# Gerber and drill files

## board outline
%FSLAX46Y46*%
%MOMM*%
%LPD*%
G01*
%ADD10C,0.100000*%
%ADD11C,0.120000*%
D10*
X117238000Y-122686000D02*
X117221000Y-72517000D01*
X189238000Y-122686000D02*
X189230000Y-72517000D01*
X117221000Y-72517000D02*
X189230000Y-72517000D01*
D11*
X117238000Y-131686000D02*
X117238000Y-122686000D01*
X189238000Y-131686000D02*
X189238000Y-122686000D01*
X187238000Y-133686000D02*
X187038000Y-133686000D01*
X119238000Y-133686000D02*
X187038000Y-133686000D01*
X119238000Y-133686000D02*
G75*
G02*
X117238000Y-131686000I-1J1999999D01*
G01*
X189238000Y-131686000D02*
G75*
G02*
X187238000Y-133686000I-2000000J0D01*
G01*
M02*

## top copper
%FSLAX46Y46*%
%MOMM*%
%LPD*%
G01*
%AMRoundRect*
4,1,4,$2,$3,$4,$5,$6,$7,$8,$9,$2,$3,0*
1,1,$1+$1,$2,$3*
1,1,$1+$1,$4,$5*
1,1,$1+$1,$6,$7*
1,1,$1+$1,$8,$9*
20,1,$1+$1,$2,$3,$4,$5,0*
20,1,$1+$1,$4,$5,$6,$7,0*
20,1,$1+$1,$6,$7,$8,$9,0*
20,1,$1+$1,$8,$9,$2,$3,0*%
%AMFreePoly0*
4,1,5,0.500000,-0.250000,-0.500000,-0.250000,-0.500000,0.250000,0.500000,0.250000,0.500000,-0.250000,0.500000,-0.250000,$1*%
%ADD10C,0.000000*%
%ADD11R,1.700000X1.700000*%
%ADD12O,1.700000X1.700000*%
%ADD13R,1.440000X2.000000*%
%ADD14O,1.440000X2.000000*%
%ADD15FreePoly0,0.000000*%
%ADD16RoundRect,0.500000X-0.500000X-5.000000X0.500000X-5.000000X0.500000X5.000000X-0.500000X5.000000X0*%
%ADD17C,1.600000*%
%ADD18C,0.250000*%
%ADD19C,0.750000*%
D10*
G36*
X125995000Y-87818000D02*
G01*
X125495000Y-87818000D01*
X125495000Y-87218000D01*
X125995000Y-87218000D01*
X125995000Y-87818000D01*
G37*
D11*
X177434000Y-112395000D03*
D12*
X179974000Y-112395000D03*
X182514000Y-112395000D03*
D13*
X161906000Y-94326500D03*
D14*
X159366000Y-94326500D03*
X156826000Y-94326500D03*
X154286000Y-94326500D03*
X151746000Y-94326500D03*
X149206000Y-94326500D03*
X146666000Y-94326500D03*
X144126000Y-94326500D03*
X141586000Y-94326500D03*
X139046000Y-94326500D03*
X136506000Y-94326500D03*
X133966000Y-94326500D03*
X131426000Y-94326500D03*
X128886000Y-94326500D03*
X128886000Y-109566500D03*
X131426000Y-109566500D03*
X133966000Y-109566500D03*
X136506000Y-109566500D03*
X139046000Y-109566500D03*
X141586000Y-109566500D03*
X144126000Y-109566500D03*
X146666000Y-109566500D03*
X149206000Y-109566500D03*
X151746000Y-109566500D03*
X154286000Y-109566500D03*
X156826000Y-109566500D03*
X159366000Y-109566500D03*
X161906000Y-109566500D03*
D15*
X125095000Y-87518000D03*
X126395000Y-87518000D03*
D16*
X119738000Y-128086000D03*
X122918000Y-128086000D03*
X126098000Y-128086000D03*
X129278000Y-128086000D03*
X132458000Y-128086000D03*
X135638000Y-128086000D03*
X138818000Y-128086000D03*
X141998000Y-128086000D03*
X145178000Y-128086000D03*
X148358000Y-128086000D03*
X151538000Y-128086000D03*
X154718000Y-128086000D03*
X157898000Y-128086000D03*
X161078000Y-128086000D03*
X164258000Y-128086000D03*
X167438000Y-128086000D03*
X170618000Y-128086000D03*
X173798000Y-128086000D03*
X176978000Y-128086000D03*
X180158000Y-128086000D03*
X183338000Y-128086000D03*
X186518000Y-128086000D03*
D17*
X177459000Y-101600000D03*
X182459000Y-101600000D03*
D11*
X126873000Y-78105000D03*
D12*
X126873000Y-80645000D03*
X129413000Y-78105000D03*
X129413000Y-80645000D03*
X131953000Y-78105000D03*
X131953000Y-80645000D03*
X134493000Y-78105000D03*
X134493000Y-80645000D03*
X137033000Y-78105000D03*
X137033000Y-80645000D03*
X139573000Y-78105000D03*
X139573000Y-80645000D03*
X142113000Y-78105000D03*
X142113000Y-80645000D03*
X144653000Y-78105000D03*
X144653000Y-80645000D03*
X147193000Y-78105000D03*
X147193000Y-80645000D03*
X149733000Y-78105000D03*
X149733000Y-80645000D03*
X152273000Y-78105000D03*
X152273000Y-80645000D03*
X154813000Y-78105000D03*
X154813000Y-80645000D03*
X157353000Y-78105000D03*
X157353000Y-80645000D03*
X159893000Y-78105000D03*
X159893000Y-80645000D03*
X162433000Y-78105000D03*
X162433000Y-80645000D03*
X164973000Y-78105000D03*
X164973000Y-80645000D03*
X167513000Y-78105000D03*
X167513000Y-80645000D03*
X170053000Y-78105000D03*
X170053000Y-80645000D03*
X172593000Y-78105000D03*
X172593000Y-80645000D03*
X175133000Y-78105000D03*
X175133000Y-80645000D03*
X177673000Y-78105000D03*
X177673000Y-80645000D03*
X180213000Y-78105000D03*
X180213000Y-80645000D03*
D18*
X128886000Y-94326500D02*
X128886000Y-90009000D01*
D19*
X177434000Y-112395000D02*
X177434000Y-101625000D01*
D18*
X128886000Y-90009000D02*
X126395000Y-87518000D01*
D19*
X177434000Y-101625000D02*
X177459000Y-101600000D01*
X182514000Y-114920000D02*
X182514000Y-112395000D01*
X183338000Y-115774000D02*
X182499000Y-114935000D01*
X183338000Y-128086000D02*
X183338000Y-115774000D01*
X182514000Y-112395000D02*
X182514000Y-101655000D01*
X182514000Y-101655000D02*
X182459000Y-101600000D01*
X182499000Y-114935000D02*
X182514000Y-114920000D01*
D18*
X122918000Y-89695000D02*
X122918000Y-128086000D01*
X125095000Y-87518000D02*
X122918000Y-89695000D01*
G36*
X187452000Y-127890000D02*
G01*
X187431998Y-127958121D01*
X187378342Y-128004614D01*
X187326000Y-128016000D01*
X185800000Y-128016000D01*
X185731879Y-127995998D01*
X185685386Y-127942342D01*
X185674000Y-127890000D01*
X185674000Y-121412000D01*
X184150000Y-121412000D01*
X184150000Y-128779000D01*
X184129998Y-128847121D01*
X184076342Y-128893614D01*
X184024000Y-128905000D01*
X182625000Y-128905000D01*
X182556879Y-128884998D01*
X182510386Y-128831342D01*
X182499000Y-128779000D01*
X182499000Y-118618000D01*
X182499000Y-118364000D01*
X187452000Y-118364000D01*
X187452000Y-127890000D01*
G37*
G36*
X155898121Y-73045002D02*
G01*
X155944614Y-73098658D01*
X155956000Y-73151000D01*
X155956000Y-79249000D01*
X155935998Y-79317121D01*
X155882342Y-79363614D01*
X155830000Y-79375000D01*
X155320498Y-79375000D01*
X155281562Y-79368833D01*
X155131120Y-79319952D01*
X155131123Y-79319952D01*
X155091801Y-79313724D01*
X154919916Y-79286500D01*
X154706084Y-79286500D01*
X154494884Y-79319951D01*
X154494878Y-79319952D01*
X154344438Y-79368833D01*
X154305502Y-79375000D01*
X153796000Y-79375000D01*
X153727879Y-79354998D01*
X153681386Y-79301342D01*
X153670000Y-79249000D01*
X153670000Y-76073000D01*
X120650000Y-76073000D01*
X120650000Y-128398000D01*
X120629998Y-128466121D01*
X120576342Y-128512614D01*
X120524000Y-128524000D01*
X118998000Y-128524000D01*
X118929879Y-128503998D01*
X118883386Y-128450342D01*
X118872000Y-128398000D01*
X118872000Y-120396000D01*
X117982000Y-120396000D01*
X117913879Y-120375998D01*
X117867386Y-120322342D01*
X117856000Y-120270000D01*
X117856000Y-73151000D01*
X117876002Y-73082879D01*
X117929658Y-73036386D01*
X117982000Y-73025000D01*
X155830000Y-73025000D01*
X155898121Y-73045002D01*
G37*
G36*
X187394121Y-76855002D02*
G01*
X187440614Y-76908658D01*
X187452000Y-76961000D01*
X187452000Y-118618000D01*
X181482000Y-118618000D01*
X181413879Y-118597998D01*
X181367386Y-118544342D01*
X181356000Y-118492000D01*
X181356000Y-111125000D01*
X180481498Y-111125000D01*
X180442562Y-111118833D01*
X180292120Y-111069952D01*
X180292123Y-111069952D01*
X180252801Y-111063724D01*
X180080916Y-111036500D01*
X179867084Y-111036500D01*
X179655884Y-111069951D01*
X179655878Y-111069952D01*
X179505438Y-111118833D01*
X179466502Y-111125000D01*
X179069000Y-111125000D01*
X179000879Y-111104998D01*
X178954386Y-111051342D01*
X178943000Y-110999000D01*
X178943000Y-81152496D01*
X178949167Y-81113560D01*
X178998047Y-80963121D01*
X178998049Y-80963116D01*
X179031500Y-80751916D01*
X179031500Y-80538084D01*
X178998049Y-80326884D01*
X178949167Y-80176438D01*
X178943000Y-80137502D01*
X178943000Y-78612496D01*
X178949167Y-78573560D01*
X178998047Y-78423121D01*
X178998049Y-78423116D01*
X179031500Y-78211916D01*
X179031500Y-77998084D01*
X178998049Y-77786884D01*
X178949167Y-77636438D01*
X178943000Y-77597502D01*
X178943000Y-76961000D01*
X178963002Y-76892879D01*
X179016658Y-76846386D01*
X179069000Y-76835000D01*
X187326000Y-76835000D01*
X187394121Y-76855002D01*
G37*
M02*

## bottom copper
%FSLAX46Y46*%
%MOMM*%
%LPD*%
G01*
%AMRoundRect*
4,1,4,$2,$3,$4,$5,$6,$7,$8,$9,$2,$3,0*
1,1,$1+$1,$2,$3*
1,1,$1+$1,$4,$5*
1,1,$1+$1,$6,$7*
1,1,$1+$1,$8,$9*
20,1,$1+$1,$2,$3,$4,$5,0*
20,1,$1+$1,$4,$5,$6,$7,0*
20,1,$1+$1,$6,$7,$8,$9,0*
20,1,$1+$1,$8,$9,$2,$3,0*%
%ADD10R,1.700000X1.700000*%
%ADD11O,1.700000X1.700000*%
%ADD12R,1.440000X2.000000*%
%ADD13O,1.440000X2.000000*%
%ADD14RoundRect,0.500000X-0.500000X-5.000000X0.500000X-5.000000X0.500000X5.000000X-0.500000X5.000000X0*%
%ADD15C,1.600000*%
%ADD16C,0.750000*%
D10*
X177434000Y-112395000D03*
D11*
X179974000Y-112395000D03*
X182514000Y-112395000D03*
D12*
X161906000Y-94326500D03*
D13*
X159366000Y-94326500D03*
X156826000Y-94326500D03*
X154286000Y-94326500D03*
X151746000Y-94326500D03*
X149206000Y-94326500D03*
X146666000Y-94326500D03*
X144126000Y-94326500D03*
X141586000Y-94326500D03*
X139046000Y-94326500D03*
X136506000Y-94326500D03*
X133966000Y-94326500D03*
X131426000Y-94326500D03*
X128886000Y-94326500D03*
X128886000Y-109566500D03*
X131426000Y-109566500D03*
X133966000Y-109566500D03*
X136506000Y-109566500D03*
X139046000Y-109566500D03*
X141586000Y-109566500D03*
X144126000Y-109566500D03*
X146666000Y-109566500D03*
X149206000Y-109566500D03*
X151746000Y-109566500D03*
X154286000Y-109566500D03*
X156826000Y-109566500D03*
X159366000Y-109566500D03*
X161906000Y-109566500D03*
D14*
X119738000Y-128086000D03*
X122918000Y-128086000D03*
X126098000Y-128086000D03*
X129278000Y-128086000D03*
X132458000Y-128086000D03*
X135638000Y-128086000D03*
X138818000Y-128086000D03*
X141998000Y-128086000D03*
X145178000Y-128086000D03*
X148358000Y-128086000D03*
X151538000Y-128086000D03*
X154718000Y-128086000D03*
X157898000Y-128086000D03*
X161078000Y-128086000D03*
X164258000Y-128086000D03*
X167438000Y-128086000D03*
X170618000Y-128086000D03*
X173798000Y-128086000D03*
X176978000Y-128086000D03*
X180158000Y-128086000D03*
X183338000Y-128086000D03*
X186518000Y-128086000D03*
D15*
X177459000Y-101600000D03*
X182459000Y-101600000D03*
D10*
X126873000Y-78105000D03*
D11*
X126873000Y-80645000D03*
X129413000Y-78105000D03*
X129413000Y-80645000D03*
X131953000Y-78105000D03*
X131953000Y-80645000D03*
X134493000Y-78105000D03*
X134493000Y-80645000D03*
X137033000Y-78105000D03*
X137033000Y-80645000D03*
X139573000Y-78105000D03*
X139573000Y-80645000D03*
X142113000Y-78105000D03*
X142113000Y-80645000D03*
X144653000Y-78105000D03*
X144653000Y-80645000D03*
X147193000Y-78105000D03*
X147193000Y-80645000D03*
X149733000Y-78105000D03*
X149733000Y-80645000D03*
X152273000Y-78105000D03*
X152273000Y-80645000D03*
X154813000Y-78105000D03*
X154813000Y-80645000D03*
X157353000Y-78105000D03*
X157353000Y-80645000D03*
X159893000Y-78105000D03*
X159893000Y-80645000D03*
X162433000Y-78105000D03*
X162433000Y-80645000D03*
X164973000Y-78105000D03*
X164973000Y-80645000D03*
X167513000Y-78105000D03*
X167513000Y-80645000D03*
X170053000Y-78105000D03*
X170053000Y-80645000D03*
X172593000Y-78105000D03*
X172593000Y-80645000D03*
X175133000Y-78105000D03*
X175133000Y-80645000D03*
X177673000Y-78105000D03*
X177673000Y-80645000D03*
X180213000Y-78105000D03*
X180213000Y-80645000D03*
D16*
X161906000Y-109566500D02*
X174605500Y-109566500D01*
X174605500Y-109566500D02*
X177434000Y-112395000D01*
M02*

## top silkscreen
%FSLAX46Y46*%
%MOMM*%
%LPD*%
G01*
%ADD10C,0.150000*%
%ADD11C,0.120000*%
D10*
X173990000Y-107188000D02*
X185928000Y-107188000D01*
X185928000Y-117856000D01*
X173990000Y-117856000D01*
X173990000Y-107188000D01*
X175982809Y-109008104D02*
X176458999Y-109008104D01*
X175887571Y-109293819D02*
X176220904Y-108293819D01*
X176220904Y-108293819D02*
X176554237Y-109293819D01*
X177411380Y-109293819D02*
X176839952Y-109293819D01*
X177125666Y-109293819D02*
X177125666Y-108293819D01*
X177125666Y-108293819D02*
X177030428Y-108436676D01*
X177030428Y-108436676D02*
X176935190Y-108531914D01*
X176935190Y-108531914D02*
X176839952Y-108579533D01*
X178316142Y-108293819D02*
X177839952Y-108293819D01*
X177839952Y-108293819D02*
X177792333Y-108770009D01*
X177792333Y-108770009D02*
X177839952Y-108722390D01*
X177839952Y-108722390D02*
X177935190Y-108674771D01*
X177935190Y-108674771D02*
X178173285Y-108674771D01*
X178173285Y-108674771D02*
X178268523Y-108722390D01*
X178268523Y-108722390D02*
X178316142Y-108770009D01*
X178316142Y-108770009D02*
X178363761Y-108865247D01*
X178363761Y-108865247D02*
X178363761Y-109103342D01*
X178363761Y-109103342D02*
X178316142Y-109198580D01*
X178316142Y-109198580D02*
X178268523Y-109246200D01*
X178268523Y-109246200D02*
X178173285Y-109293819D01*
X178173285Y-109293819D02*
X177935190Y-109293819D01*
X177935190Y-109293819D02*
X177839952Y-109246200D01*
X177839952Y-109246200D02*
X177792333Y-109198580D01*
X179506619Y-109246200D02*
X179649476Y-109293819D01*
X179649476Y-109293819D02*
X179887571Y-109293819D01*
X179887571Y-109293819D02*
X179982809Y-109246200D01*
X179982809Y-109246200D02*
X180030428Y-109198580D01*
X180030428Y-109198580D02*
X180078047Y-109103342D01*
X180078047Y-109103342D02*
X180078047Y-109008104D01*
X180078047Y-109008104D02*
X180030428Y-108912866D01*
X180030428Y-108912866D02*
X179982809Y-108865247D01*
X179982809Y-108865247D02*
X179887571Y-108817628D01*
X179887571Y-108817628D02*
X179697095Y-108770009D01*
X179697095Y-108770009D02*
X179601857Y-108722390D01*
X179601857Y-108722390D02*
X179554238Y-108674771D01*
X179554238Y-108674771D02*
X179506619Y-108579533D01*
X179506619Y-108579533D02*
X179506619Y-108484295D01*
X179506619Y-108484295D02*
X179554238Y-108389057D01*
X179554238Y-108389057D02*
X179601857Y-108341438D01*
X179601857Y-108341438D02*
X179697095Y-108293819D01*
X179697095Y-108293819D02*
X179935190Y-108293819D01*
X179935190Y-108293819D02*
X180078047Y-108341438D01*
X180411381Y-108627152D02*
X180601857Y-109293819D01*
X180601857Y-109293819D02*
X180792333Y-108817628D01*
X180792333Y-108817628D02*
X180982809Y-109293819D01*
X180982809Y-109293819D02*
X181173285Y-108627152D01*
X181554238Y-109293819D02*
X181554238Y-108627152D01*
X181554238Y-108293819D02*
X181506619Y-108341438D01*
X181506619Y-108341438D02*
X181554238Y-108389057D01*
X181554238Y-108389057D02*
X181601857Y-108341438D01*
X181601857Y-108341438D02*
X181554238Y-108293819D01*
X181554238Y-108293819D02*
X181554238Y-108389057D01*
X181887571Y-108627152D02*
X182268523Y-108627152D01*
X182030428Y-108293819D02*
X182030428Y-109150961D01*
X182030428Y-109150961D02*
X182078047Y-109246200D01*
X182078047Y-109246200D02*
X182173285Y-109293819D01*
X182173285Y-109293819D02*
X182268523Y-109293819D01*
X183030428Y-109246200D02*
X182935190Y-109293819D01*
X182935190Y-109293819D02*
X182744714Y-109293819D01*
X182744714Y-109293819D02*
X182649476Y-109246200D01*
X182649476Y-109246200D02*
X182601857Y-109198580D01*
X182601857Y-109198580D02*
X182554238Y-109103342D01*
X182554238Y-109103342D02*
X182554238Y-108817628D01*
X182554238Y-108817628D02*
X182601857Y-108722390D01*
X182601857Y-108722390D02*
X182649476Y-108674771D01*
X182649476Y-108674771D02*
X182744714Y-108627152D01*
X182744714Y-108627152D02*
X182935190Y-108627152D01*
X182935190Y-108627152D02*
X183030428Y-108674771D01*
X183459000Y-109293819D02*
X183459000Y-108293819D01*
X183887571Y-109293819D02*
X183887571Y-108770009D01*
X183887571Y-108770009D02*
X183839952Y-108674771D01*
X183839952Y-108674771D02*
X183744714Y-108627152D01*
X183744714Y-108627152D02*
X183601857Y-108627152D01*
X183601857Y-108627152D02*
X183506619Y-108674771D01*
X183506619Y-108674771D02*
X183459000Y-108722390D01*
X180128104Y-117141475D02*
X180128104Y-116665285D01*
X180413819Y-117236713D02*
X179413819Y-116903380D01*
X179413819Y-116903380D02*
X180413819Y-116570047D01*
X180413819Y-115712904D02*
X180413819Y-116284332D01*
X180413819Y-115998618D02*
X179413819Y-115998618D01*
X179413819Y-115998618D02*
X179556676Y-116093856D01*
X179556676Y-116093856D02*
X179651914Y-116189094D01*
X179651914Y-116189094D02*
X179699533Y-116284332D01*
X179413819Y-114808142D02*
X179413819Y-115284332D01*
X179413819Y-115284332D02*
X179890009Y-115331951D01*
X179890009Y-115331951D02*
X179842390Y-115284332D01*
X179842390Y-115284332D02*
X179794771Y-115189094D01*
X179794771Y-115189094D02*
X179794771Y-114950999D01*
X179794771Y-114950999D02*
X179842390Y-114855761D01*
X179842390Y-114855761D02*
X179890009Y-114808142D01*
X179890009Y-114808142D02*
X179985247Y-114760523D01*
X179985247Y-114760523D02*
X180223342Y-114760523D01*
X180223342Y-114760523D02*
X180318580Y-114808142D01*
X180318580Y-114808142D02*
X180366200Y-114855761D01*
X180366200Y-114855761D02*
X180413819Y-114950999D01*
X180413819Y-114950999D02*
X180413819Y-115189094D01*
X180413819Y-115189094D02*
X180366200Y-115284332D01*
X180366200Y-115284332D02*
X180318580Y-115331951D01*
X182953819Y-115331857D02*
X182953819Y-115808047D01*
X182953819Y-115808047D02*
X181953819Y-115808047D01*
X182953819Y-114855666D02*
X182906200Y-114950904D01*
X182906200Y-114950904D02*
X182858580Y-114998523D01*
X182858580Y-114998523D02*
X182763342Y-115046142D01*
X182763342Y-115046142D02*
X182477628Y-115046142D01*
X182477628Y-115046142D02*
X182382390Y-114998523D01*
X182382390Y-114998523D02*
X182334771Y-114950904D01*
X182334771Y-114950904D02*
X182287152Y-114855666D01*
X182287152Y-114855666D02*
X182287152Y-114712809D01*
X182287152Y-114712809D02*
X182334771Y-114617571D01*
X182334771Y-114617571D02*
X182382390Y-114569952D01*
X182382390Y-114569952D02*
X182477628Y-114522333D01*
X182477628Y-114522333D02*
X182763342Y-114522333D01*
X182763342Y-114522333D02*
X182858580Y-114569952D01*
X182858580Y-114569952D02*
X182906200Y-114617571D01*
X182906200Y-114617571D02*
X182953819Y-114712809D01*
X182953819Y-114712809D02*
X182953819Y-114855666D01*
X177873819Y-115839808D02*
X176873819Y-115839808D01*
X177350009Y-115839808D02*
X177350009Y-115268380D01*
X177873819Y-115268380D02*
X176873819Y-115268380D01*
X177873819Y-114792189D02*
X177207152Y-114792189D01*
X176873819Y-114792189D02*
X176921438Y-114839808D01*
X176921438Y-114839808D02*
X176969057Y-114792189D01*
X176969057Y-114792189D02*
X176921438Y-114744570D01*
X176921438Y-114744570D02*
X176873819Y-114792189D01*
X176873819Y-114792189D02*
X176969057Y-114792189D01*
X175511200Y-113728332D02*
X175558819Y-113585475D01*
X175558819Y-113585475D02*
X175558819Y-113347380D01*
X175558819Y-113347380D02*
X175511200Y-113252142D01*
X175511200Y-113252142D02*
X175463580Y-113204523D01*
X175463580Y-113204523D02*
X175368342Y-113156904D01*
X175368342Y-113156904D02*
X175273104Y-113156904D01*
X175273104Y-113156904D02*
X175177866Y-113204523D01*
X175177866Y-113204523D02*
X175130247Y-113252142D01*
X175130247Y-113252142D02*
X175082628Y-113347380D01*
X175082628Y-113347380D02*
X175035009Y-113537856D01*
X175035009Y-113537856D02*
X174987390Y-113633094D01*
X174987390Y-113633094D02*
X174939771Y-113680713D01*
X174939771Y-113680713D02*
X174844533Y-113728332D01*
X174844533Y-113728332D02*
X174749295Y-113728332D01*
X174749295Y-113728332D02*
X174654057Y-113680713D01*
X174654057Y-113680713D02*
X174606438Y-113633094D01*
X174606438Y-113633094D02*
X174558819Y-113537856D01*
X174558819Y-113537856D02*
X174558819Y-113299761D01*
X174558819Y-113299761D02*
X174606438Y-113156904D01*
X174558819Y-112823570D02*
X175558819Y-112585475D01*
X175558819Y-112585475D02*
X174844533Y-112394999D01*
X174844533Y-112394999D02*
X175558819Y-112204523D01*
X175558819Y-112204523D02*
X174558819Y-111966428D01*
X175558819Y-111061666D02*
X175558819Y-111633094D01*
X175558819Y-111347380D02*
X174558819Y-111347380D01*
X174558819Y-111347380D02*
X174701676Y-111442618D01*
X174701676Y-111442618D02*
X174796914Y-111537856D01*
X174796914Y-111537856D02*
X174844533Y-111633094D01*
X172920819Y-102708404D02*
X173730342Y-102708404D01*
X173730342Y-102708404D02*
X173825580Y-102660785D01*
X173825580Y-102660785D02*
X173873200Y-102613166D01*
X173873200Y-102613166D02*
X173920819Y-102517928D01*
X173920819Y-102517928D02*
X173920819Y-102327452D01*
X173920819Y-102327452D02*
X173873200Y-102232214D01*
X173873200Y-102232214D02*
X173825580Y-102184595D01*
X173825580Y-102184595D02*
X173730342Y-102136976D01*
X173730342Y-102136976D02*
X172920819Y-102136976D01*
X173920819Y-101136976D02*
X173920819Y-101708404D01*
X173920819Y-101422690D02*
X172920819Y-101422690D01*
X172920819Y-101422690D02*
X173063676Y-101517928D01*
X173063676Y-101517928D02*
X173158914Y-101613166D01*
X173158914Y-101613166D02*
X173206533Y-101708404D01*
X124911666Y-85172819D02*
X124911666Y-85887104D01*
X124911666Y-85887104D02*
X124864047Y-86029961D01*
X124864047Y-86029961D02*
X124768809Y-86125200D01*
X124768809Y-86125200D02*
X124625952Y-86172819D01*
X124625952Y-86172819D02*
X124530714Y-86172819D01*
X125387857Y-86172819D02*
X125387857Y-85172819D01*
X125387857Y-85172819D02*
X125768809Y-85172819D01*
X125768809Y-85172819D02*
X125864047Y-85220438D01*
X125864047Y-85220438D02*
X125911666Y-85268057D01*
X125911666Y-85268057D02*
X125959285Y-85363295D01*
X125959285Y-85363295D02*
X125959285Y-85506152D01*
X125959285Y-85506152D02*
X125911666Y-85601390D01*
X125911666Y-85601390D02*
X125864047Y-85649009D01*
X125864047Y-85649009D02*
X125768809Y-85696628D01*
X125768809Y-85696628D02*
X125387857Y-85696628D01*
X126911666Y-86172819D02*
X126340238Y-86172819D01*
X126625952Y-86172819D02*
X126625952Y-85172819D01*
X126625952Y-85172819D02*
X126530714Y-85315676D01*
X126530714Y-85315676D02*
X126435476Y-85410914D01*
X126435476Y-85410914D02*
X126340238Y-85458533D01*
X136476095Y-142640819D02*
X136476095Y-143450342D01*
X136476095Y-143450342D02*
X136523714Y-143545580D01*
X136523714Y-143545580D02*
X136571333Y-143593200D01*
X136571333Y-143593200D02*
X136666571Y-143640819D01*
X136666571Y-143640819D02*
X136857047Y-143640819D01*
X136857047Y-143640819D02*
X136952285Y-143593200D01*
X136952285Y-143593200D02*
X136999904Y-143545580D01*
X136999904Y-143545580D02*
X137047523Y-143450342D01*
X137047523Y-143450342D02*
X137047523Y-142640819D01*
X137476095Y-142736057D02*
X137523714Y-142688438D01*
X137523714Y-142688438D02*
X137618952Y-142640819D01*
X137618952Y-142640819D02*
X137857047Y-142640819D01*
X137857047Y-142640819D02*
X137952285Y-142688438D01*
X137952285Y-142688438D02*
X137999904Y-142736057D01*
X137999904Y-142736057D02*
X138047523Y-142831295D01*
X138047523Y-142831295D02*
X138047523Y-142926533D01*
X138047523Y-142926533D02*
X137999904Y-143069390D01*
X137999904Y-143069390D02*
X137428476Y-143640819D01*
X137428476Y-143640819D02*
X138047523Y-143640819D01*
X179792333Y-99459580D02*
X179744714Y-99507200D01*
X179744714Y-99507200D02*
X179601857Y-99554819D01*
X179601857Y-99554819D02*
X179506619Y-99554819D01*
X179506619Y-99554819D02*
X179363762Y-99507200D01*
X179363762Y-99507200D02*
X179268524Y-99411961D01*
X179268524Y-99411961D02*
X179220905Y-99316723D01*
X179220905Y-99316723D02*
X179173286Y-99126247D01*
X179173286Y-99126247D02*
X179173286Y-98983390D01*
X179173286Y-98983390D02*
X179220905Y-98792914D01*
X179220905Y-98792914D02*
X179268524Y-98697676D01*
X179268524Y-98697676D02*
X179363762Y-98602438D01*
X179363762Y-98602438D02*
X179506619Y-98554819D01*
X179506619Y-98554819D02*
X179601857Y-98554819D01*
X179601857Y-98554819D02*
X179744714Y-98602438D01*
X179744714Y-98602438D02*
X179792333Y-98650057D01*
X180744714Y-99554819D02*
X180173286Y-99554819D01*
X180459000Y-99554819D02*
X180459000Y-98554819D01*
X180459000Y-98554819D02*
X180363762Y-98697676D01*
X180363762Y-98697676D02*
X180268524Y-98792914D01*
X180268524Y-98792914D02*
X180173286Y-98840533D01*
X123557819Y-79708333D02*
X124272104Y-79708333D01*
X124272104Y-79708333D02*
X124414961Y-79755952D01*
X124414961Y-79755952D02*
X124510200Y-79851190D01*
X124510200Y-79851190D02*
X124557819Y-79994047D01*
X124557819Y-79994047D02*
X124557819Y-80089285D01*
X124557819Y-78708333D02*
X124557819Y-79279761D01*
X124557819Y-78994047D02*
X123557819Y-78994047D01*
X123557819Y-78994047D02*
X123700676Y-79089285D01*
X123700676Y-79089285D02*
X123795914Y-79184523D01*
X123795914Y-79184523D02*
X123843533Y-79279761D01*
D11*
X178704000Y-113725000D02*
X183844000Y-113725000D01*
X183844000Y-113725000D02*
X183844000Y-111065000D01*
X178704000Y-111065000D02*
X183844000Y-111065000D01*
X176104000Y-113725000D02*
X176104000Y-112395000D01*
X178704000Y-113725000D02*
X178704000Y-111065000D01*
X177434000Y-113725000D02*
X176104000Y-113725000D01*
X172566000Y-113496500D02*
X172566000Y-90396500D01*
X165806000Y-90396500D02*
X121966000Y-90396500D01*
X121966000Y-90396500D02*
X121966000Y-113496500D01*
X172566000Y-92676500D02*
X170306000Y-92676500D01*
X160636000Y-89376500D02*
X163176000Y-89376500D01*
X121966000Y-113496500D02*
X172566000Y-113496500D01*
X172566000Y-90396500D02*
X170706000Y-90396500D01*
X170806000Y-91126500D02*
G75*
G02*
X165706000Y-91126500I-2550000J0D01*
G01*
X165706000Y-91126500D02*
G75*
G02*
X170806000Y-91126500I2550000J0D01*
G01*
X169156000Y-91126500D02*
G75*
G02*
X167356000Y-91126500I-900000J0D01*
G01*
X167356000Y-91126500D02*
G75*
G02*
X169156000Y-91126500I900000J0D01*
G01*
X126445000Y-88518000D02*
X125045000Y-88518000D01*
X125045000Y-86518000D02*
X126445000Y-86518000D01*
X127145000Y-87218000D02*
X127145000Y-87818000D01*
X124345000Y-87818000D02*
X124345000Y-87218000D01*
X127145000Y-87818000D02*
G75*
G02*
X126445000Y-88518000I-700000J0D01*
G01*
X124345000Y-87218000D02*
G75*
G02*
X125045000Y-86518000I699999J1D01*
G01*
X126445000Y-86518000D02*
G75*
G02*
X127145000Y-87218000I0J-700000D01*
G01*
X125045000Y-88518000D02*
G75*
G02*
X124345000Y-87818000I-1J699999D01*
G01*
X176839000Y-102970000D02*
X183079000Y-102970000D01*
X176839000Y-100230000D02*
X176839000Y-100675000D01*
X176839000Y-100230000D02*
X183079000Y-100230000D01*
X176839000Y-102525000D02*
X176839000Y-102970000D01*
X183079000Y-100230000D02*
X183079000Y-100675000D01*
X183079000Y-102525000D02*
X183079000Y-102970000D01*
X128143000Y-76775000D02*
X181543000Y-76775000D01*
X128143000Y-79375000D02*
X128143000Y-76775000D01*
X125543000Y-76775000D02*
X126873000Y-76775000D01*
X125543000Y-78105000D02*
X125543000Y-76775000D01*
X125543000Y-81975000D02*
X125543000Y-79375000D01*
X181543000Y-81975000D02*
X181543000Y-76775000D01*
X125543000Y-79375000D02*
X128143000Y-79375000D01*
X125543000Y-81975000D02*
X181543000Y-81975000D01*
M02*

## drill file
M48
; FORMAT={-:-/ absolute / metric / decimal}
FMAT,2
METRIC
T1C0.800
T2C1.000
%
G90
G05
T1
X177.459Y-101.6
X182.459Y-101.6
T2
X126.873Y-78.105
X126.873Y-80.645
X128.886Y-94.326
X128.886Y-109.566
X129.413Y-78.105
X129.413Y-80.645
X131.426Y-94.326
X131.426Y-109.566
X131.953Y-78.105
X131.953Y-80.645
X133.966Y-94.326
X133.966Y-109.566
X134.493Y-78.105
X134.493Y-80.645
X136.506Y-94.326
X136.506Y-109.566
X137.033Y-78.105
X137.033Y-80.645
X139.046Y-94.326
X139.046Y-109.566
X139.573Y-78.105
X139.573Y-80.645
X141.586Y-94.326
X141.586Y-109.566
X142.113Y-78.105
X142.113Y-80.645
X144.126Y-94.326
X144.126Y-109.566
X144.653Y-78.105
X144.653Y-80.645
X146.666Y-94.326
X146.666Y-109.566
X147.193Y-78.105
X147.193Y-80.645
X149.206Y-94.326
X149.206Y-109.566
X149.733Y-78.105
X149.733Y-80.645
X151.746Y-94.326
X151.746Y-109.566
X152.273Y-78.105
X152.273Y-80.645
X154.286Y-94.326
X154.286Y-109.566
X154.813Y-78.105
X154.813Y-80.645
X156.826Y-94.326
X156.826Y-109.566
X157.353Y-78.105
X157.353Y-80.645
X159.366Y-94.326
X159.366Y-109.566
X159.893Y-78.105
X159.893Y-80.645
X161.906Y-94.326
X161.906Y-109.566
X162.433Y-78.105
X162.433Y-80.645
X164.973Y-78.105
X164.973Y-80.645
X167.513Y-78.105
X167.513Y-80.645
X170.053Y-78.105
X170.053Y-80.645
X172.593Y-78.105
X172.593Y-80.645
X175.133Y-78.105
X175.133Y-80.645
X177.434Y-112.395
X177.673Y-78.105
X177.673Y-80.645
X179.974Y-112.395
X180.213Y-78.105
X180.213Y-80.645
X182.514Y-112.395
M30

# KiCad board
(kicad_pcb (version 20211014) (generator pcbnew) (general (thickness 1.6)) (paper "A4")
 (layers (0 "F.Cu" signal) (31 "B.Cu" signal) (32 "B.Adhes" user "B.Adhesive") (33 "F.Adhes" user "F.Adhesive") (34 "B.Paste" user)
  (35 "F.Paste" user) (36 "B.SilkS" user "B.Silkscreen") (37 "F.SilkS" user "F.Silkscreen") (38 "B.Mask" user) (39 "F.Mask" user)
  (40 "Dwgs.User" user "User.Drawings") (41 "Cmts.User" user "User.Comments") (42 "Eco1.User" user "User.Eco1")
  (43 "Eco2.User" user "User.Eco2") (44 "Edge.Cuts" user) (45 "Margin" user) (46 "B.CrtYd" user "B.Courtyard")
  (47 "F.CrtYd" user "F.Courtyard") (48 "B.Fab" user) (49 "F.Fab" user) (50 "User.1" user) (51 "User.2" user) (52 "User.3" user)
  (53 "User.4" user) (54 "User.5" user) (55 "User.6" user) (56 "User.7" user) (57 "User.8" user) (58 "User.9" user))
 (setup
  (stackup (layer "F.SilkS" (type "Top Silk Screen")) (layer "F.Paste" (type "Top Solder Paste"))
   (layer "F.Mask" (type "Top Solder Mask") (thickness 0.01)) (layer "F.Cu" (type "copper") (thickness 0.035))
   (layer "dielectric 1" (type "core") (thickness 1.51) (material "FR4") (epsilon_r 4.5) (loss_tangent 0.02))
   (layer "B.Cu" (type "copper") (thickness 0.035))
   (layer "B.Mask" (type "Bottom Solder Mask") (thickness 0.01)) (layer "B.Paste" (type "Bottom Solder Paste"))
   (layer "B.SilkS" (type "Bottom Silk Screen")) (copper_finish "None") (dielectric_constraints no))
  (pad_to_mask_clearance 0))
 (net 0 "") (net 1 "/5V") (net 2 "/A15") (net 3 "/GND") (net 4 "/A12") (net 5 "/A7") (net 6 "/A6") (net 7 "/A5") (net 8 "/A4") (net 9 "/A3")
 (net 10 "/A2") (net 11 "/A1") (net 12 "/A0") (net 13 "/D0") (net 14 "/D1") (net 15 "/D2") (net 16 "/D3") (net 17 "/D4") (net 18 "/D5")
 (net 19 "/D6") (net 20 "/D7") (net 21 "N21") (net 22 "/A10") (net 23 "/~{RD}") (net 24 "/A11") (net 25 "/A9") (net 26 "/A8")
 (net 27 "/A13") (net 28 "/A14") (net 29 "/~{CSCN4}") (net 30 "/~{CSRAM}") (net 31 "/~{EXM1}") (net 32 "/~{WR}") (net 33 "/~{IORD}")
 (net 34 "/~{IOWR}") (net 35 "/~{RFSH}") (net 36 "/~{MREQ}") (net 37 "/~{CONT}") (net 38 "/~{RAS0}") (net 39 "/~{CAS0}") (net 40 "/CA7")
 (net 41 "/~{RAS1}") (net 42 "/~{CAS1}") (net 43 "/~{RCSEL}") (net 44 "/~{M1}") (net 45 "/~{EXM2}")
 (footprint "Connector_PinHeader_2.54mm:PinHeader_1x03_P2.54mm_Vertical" (layer "F.Cu") (at 177.434 112.395 90)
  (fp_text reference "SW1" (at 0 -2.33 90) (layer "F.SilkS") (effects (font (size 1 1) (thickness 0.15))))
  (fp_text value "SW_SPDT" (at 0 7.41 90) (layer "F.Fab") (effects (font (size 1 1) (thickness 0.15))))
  (fp_line (start -1.33 1.27) (end -1.33 6.41) (layer "F.SilkS") (width 0.12))
  (fp_line (start -1.33 6.41) (end 1.33 6.41) (layer "F.SilkS") (width 0.12))
  (fp_line (start 1.33 1.27) (end 1.33 6.41) (layer "F.SilkS") (width 0.12))
  (fp_line (start -1.33 -1.33) (end 0 -1.33) (layer "F.SilkS") (width 0.12))
  (fp_line (start -1.33 1.27) (end 1.33 1.27) (layer "F.SilkS") (width 0.12))
  (fp_line (start -1.33 0) (end -1.33 -1.33) (layer "F.SilkS") (width 0.12))
  (pad "1" thru_hole rect (at 0 0 90) (size 1.7 1.7) (drill 1) (layers *.Cu *.Mask) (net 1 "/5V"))
  (pad "2" thru_hole oval (at 0 2.54 90) (size 1.7 1.7) (drill 1) (layers *.Cu *.Mask) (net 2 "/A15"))
  (pad "3" thru_hole oval (at 0 5.08 90) (size 1.7 1.7) (drill 1) (layers *.Cu *.Mask) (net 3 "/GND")))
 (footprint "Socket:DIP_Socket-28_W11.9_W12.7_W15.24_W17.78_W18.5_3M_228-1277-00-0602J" (layer "F.Cu") (at 161.906 94.3265 -90)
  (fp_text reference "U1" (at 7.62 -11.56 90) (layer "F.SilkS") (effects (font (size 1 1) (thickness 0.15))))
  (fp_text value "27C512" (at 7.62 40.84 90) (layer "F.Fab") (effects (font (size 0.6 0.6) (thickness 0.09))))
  (fp_line (start 19.17 -10.66) (end -3.93 -10.66) (layer "F.SilkS") (width 0.12))
  (fp_line (start -3.93 -3.9) (end -3.93 39.94) (layer "F.SilkS") (width 0.12))
  (fp_line (start -3.93 39.94) (end 19.17 39.94) (layer "F.SilkS") (width 0.12))
  (fp_line (start -1.65 -10.66) (end -1.65 -8.4) (layer "F.SilkS") (width 0.12))
  (fp_line (start -4.95 1.27) (end -4.95 -1.27) (layer "F.SilkS") (width 0.12))
  (fp_line (start 19.17 39.94) (end 19.17 -10.66) (layer "F.SilkS") (width 0.12))
  (fp_line (start -3.93 -10.66) (end -3.93 -8.8) (layer "F.SilkS") (width 0.12))
  (fp_circle (center -3.2 -6.35) (end -0.65 -6.35) (layer "F.SilkS") (width 0.12) (fill none))
  (fp_circle (center -3.2 -6.35) (end -2.3 -6.35) (layer "F.SilkS") (width 0.12) (fill none))
  (pad "1" thru_hole rect (at 0 0 270) (size 2 1.44) (drill 1) (layers *.Cu *.Mask) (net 2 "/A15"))
  (pad "2" thru_hole oval (at 0 2.54 270) (size 2 1.44) (drill 1) (layers *.Cu *.Mask) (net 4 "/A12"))
  (pad "3" thru_hole oval (at 0 5.08 270) (size 2 1.44) (drill 1) (layers *.Cu *.Mask) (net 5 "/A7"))
  (pad "4" thru_hole oval (at 0 7.62 270) (size 2 1.44) (drill 1) (layers *.Cu *.Mask) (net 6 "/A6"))
  (pad "5" thru_hole oval (at 0 10.16 270) (size 2 1.44) (drill 1) (layers *.Cu *.Mask) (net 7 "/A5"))
  (pad "6" thru_hole oval (at 0 12.7 270) (size 2 1.44) (drill 1) (layers *.Cu *.Mask) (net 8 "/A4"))
  (pad "7" thru_hole oval (at 0 15.24 270) (size 2 1.44) (drill 1) (layers *.Cu *.Mask) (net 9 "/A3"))
  (pad "8" thru_hole oval (at 0 17.78 270) (size 2 1.44) (drill 1) (layers *.Cu *.Mask) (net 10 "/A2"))
  (pad "9" thru_hole oval (at 0 20.32 270) (size 2 1.44) (drill 1) (layers *.Cu *.Mask) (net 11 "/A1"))
  (pad "10" thru_hole oval (at 0 22.86 270) (size 2 1.44) (drill 1) (layers *.Cu *.Mask) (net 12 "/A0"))
  (pad "11" thru_hole oval (at 0 25.4 270) (size 2 1.44) (drill 1) (layers *.Cu *.Mask) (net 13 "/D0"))
  (pad "12" thru_hole oval (at 0 27.94 270) (size 2 1.44) (drill 1) (layers *.Cu *.Mask) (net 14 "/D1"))
  (pad "13" thru_hole oval (at 0 30.48 270) (size 2 1.44) (drill 1) (layers *.Cu *.Mask) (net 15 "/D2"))
  (pad "14" thru_hole oval (at 0 33.02 270) (size 2 1.44) (drill 1) (layers *.Cu *.Mask) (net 3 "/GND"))
  (pad "15" thru_hole oval (at 15.24 33.02 270) (size 2 1.44) (drill 1) (layers *.Cu *.Mask) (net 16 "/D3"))
  (pad "16" thru_hole oval (at 15.24 30.48 270) (size 2 1.44) (drill 1) (layers *.Cu *.Mask) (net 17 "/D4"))
  (pad "17" thru_hole oval (at 15.24 27.94 270) (size 2 1.44) (drill 1) (layers *.Cu *.Mask) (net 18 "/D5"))
  (pad "18" thru_hole oval (at 15.24 25.4 270) (size 2 1.44) (drill 1) (layers *.Cu *.Mask) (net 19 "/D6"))
  (pad "19" thru_hole oval (at 15.24 22.86 270) (size 2 1.44) (drill 1) (layers *.Cu *.Mask) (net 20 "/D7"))
  (pad "20" thru_hole oval (at 15.24 20.32 270) (size 2 1.44) (drill 1) (layers *.Cu *.Mask) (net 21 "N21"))
  (pad "21" thru_hole oval (at 15.24 17.78 270) (size 2 1.44) (drill 1) (layers *.Cu *.Mask) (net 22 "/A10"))
  (pad "22" thru_hole oval (at 15.24 15.24 270) (size 2 1.44) (drill 1) (layers *.Cu *.Mask) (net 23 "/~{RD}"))
  (pad "23" thru_hole oval (at 15.24 12.7 270) (size 2 1.44) (drill 1) (layers *.Cu *.Mask) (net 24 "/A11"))
  (pad "24" thru_hole oval (at 15.24 10.16 270) (size 2 1.44) (drill 1) (layers *.Cu *.Mask) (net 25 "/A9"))
  (pad "25" thru_hole oval (at 15.24 7.62 270) (size 2 1.44) (drill 1) (layers *.Cu *.Mask) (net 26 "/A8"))
  (pad "26" thru_hole oval (at 15.24 5.08 270) (size 2 1.44) (drill 1) (layers *.Cu *.Mask) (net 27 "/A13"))
  (pad "27" thru_hole oval (at 15.24 2.54 270) (size 2 1.44) (drill 1) (layers *.Cu *.Mask) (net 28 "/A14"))
  (pad "28" thru_hole oval (at 15.24 0 270) (size 2 1.44) (drill 1) (layers *.Cu *.Mask) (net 1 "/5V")))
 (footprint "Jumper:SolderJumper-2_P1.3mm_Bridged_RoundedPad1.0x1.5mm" (layer "F.Cu") (at 125.745 87.518)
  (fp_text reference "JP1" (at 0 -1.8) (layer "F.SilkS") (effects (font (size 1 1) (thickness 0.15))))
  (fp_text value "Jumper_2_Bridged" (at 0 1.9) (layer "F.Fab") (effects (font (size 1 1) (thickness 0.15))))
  (fp_poly (pts (xy 0.25 -0.3) (xy -0.25 -0.3) (xy -0.25 0.3) (xy 0.25 0.3)) (layer "F.Cu") (width 0) (fill solid))
  (fp_line (start 0.7 1) (end -0.7 1) (layer "F.SilkS") (width 0.12))
  (fp_line (start -0.7 -1) (end 0.7 -1) (layer "F.SilkS") (width 0.12))
  (fp_line (start 1.4 -0.3) (end 1.4 0.3) (layer "F.SilkS") (width 0.12))
  (fp_line (start -1.4 0.3) (end -1.4 -0.3) (layer "F.SilkS") (width 0.12))
  (fp_arc (start 1.4 0.3) (mid 1.194975 0.794975) (end 0.7 1) (layer "F.SilkS") (width 0.12))
  (fp_arc (start -1.4 -0.3) (mid -1.194975 -0.794975) (end -0.7 -1) (layer "F.SilkS") (width 0.12))
  (fp_arc (start 0.7 -1) (mid 1.194975 -0.794975) (end 1.4 -0.3) (layer "F.SilkS") (width 0.12))
  (fp_arc (start -0.7 1) (mid -1.194975 0.794975) (end -1.4 0.3) (layer "F.SilkS") (width 0.12))
  (pad "1" smd custom (at -0.65 0) (size 1 0.5) (layers "F.Cu" "F.Mask") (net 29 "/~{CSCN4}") (zone_connect 2)
   (options (clearance outline) (anchor rect)) (primitives))
  (pad "2" smd custom (at 0.65 0) (size 1 0.5) (layers "F.Cu" "F.Mask") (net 1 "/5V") (zone_connect 2)
   (options (clearance outline) (anchor rect)) (primitives)))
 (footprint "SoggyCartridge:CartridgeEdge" (layer "F.Cu") (at 120.138 122.586)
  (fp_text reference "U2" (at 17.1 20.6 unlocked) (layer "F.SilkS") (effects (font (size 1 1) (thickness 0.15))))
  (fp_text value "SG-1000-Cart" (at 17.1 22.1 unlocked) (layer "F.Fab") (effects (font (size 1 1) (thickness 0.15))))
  (fp_line (start -2.9 9.1) (end -2.9 0.1) (layer "Edge.Cuts") (width 0.12))
  (fp_line (start 69.1 9.1) (end 69.1 0.1) (layer "Edge.Cuts") (width 0.12))
  (fp_line (start 67.1 11.1) (end 66.9 11.1) (layer "Edge.Cuts") (width 0.12))
  (fp_line (start -0.9 11.1) (end 66.9 11.1) (layer "Edge.Cuts") (width 0.12))
  (fp_arc (start -0.9 11.1) (mid -2.314214 10.514214) (end -2.9 9.1) (layer "Edge.Cuts") (width 0.12))
  (fp_arc (start 69.1 9.1) (mid 68.514214 10.514214) (end 67.1 11.1) (layer "Edge.Cuts") (width 0.12))
  (pad "A1" connect roundrect (at -0.4 5.5) (size 2 11) (layers "B.Cu" "B.Mask") (roundrect_rratio 0.25) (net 12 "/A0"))
  (pad "A2" connect roundrect (at 2.78 5.5) (size 2 11) (layers "B.Cu" "B.Mask") (roundrect_rratio 0.25) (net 11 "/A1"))
  (pad "A3" connect roundrect (at 5.96 5.5) (size 2 11) (layers "B.Cu" "B.Mask") (roundrect_rratio 0.25) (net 10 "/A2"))
  (pad "A4" connect roundrect (at 9.14 5.5) (size 2 11) (layers "B.Cu" "B.Mask") (roundrect_rratio 0.25) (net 9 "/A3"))
  (pad "A5" connect roundrect (at 12.32 5.5) (size 2 11) (layers "B.Cu" "B.Mask") (roundrect_rratio 0.25) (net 8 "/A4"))
  (pad "A6" connect roundrect (at 15.5 5.5) (size 2 11) (layers "B.Cu" "B.Mask") (roundrect_rratio 0.25) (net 7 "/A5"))
  (pad "A7" connect roundrect (at 18.68 5.5) (size 2 11) (layers "B.Cu" "B.Mask") (roundrect_rratio 0.25) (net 6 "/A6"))
  (pad "A8" connect roundrect (at 21.86 5.5) (size 2 11) (layers "B.Cu" "B.Mask") (roundrect_rratio 0.25) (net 5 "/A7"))
  (pad "A9" connect roundrect (at 25.04 5.5) (size 2 11) (layers "B.Cu" "B.Mask") (roundrect_rratio 0.25) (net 26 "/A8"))
  (pad "A10" connect roundrect (at 28.22 5.5) (size 2 11) (layers "B.Cu" "B.Mask") (roundrect_rratio 0.25) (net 25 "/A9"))
  (pad "A11" connect roundrect (at 31.4 5.5) (size 2 11) (layers "B.Cu" "B.Mask") (roundrect_rratio 0.25) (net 22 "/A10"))
  (pad "A12" connect roundrect (at 34.58 5.5) (size 2 11) (layers "B.Cu" "B.Mask") (roundrect_rratio 0.25) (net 24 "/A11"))
  (pad "A13" connect roundrect (at 37.76 5.5) (size 2 11) (layers "B.Cu" "B.Mask") (roundrect_rratio 0.25) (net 4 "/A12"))
  (pad "A14" connect roundrect (at 40.94 5.5) (size 2 11) (layers "B.Cu" "B.Mask") (roundrect_rratio 0.25) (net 27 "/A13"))
  (pad "A15" connect roundrect (at 44.12 5.5) (size 2 11) (layers "B.Cu" "B.Mask") (roundrect_rratio 0.25) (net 13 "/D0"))
  (pad "A16" connect roundrect (at 47.3 5.5) (size 2 11) (layers "B.Cu" "B.Mask") (roundrect_rratio 0.25) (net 14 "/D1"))
  (pad "A17" connect roundrect (at 50.48 5.5) (size 2 11) (layers "B.Cu" "B.Mask") (roundrect_rratio 0.25) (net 15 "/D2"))
  (pad "A18" connect roundrect (at 53.66 5.5) (size 2 11) (layers "B.Cu" "B.Mask") (roundrect_rratio 0.25) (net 16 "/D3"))
  (pad "A19" connect roundrect (at 56.84 5.5) (size 2 11) (layers "B.Cu" "B.Mask") (roundrect_rratio 0.25) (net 17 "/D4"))
  (pad "A20" connect roundrect (at 60.02 5.5) (size 2 11) (layers "B.Cu" "B.Mask") (roundrect_rratio 0.25) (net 18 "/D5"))
  (pad "A21" connect roundrect (at 63.2 5.5) (size 2 11) (layers "B.Cu" "B.Mask") (roundrect_rratio 0.25) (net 19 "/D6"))
  (pad "A22" connect roundrect (at 66.38 5.5) (size 2 11) (layers "B.Cu" "B.Mask") (roundrect_rratio 0.25) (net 20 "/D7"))
  (pad "B1" connect roundrect (at -0.4 5.5) (size 2 11) (layers "F.Cu" "F.Mask") (roundrect_rratio 0.25) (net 1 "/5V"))
  (pad "B2" connect roundrect (at 2.78 5.5) (size 2 11) (layers "F.Cu" "F.Mask") (roundrect_rratio 0.25) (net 29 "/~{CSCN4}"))
  (pad "B3" connect roundrect (at 5.96 5.5) (size 2 11) (layers "F.Cu" "F.Mask") (roundrect_rratio 0.25) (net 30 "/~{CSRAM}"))
  (pad "B4" connect roundrect (at 9.14 5.5) (size 2 11) (layers "F.Cu" "F.Mask") (roundrect_rratio 0.25) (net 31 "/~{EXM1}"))
  (pad "B5" connect roundrect (at 12.32 5.5) (size 2 11) (layers "F.Cu" "F.Mask") (roundrect_rratio 0.25) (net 23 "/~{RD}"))
  (pad "B6" connect roundrect (at 15.5 5.5) (size 2 11) (layers "F.Cu" "F.Mask") (roundrect_rratio 0.25) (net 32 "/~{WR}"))
  (pad "B7" connect roundrect (at 18.68 5.5) (size 2 11) (layers "F.Cu" "F.Mask") (roundrect_rratio 0.25) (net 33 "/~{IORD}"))
  (pad "B8" connect roundrect (at 21.86 5.5) (size 2 11) (layers "F.Cu" "F.Mask") (roundrect_rratio 0.25) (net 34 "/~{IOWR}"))
  (pad "B9" connect roundrect (at 25.04 5.5) (size 2 11) (layers "F.Cu" "F.Mask") (roundrect_rratio 0.25) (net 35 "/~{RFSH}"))
  (pad "B10" connect roundrect (at 28.22 5.5) (size 2 11) (layers "F.Cu" "F.Mask") (roundrect_rratio 0.25) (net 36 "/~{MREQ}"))
  (pad "B11" connect roundrect (at 31.4 5.5) (size 2 11) (layers "F.Cu" "F.Mask") (roundrect_rratio 0.25) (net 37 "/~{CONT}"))
  (pad "B12" connect roundrect (at 34.58 5.5) (size 2 11) (layers "F.Cu" "F.Mask") (roundrect_rratio 0.25) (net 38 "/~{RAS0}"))
  (pad "B13" connect roundrect (at 37.76 5.5) (size 2 11) (layers "F.Cu" "F.Mask") (roundrect_rratio 0.25) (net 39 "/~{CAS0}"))
  (pad "B14" connect roundrect (at 40.94 5.5) (size 2 11) (layers "F.Cu" "F.Mask") (roundrect_rratio 0.25) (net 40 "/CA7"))
  (pad "B15" connect roundrect (at 44.12 5.5) (size 2 11) (layers "F.Cu" "F.Mask") (roundrect_rratio 0.25) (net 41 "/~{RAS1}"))
  (pad "B16" connect roundrect (at 47.3 5.5) (size 2 11) (layers "F.Cu" "F.Mask") (roundrect_rratio 0.25) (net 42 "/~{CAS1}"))
  (pad "B17" connect roundrect (at 50.48 5.5) (size 2 11) (layers "F.Cu" "F.Mask") (roundrect_rratio 0.25) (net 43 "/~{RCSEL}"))
  (pad "B18" connect roundrect (at 53.66 5.5) (size 2 11) (layers "F.Cu" "F.Mask") (roundrect_rratio 0.25) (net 28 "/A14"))
  (pad "B19" connect roundrect (at 56.84 5.5) (size 2 11) (layers "F.Cu" "F.Mask") (roundrect_rratio 0.25) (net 21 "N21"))
  (pad "B20" connect roundrect (at 60.02 5.5) (size 2 11) (layers "F.Cu" "F.Mask") (roundrect_rratio 0.25) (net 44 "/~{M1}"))
  (pad "B21" connect roundrect (at 63.2 5.5) (size 2 11) (layers "F.Cu" "F.Mask") (roundrect_rratio 0.25) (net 3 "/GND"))
  (pad "B22" connect roundrect (at 66.38 5.5) (size 2 11) (layers "F.Cu" "F.Mask") (roundrect_rratio 0.25) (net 3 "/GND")))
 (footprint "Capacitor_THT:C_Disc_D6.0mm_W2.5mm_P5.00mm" (layer "F.Cu") (at 177.459 101.6)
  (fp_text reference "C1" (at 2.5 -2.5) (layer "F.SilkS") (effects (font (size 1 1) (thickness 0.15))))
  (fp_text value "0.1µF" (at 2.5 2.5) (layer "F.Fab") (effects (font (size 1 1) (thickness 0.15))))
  (fp_line (start -0.62 1.37) (end 5.62 1.37) (layer "F.SilkS") (width 0.12))
  (fp_line (start -0.62 -1.37) (end -0.62 -0.925) (layer "F.SilkS") (width 0.12))
  (fp_line (start -0.62 -1.37) (end 5.62 -1.37) (layer "F.SilkS") (width 0.12))
  (fp_line (start -0.62 0.925) (end -0.62 1.37) (layer "F.SilkS") (width 0.12))
  (fp_line (start 5.62 -1.37) (end 5.62 -0.925) (layer "F.SilkS") (width 0.12))
  (fp_line (start 5.62 0.925) (end 5.62 1.37) (layer "F.SilkS") (width 0.12))
  (pad "1" thru_hole circle (at 0 0) (size 1.6 1.6) (drill 0.8) (layers *.Cu *.Mask) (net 1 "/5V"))
  (pad "2" thru_hole circle (at 5 0) (size 1.6 1.6) (drill 0.8) (layers *.Cu *.Mask) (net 3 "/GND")))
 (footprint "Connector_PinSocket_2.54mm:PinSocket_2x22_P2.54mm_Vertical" (layer "F.Cu") (at 126.873 78.105 90)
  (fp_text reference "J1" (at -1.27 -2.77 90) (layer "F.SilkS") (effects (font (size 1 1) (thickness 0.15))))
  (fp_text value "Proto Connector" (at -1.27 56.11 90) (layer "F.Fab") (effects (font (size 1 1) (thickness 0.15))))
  (fp_line (start 1.33 1.27) (end 1.33 54.67) (layer "F.SilkS") (width 0.12))
  (fp_line (start -1.27 1.27) (end 1.33 1.27) (layer "F.SilkS") (width 0.12))
  (fp_line (start 1.33 -1.33) (end 1.33 0) (layer "F.SilkS") (width 0.12))
  (fp_line (start 0 -1.33) (end 1.33 -1.33) (layer "F.SilkS") (width 0.12))
  (fp_line (start -3.87 -1.33) (end -1.27 -1.33) (layer "F.SilkS") (width 0.12))
  (fp_line (start -3.87 54.67) (end 1.33 54.67) (layer "F.SilkS") (width 0.12))
  (fp_line (start -1.27 -1.33) (end -1.27 1.27) (layer "F.SilkS") (width 0.12))
  (fp_line (start -3.87 -1.33) (end -3.87 54.67) (layer "F.SilkS") (width 0.12))
  (pad "1" thru_hole rect (at 0 0 90) (size 1.7 1.7) (drill 1) (layers *.Cu *.Mask) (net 12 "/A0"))
  (pad "2" thru_hole oval (at -2.54 0 90) (size 1.7 1.7) (drill 1) (layers *.Cu *.Mask) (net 11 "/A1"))
  (pad "3" thru_hole oval (at 0 2.54 90) (size 1.7 1.7) (drill 1) (layers *.Cu *.Mask) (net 10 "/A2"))
  (pad "4" thru_hole oval (at -2.54 2.54 90) (size 1.7 1.7) (drill 1) (layers *.Cu *.Mask) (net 9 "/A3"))
  (pad "5" thru_hole oval (at 0 5.08 90) (size 1.7 1.7) (drill 1) (layers *.Cu *.Mask) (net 8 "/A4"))
  (pad "6" thru_hole oval (at -2.54 5.08 90) (size 1.7 1.7) (drill 1) (layers *.Cu *.Mask) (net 7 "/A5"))
  (pad "7" thru_hole oval (at 0 7.62 90) (size 1.7 1.7) (drill 1) (layers *.Cu *.Mask) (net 6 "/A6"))
  (pad "8" thru_hole oval (at -2.54 7.62 90) (size 1.7 1.7) (drill 1) (layers *.Cu *.Mask) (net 5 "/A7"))
  (pad "9" thru_hole oval (at 0 10.16 90) (size 1.7 1.7) (drill 1) (layers *.Cu *.Mask) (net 26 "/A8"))
  (pad "10" thru_hole oval (at -2.54 10.16 90) (size 1.7 1.7) (drill 1) (layers *.Cu *.Mask) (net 25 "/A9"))
  (pad "11" thru_hole oval (at 0 12.7 90) (size 1.7 1.7) (drill 1) (layers *.Cu *.Mask) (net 22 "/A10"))
  (pad "12" thru_hole oval (at -2.54 12.7 90) (size 1.7 1.7) (drill 1) (layers *.Cu *.Mask) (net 24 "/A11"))
  (pad "13" thru_hole oval (at 0 15.24 90) (size 1.7 1.7) (drill 1) (layers *.Cu *.Mask) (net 4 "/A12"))
  (pad "14" thru_hole oval (at -2.54 15.24 90) (size 1.7 1.7) (drill 1) (layers *.Cu *.Mask) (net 27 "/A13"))
  (pad "15" thru_hole oval (at 0 17.78 90) (size 1.7 1.7) (drill 1) (layers *.Cu *.Mask) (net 13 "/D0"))
  (pad "16" thru_hole oval (at -2.54 17.78 90) (size 1.7 1.7) (drill 1) (layers *.Cu *.Mask) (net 14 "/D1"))
  (pad "17" thru_hole oval (at 0 20.32 90) (size 1.7 1.7) (drill 1) (layers *.Cu *.Mask) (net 15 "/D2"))
  (pad "18" thru_hole oval (at -2.54 20.32 90) (size 1.7 1.7) (drill 1) (layers *.Cu *.Mask) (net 16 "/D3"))
  (pad "19" thru_hole oval (at 0 22.86 90) (size 1.7 1.7) (drill 1) (layers *.Cu *.Mask) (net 17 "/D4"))
  (pad "20" thru_hole oval (at -2.54 22.86 90) (size 1.7 1.7) (drill 1) (layers *.Cu *.Mask) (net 18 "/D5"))
  (pad "21" thru_hole oval (at 0 25.4 90) (size 1.7 1.7) (drill 1) (layers *.Cu *.Mask) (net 19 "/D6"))
  (pad "22" thru_hole oval (at -2.54 25.4 90) (size 1.7 1.7) (drill 1) (layers *.Cu *.Mask) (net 20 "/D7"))
  (pad "23" thru_hole oval (at 0 27.94 90) (size 1.7 1.7) (drill 1) (layers *.Cu *.Mask) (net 1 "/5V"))
  (pad "24" thru_hole oval (at -2.54 27.94 90) (size 1.7 1.7) (drill 1) (layers *.Cu *.Mask) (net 29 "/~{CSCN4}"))
  (pad "25" thru_hole oval (at 0 30.48 90) (size 1.7 1.7) (drill 1) (layers *.Cu *.Mask) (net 30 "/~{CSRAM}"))
  (pad "26" thru_hole oval (at -2.54 30.48 90) (size 1.7 1.7) (drill 1) (layers *.Cu *.Mask) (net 31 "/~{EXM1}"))
  (pad "27" thru_hole oval (at 0 33.02 90) (size 1.7 1.7) (drill 1) (layers *.Cu *.Mask) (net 23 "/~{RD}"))
  (pad "28" thru_hole oval (at -2.54 33.02 90) (size 1.7 1.7) (drill 1) (layers *.Cu *.Mask) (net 32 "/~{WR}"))
  (pad "29" thru_hole oval (at 0 35.56 90) (size 1.7 1.7) (drill 1) (layers *.Cu *.Mask) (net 33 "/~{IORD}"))
  (pad "30" thru_hole oval (at -2.54 35.56 90) (size 1.7 1.7) (drill 1) (layers *.Cu *.Mask) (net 34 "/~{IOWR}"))
  (pad "31" thru_hole oval (at 0 38.1 90) (size 1.7 1.7) (drill 1) (layers *.Cu *.Mask) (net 35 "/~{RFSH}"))
  (pad "32" thru_hole oval (at -2.54 38.1 90) (size 1.7 1.7) (drill 1) (layers *.Cu *.Mask) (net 36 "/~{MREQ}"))
  (pad "33" thru_hole oval (at 0 40.64 90) (size 1.7 1.7) (drill 1) (layers *.Cu *.Mask) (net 37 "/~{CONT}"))
  (pad "34" thru_hole oval (at -2.54 40.64 90) (size 1.7 1.7) (drill 1) (layers *.Cu *.Mask) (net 38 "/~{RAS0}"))
  (pad "35" thru_hole oval (at 0 43.18 90) (size 1.7 1.7) (drill 1) (layers *.Cu *.Mask) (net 39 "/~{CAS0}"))
  (pad "36" thru_hole oval (at -2.54 43.18 90) (size 1.7 1.7) (drill 1) (layers *.Cu *.Mask) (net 40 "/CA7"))
  (pad "37" thru_hole oval (at 0 45.72 90) (size 1.7 1.7) (drill 1) (layers *.Cu *.Mask) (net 41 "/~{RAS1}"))
  (pad "38" thru_hole oval (at -2.54 45.72 90) (size 1.7 1.7) (drill 1) (layers *.Cu *.Mask) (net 42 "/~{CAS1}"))
  (pad "39" thru_hole oval (at 0 48.26 90) (size 1.7 1.7) (drill 1) (layers *.Cu *.Mask) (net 43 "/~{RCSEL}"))
  (pad "40" thru_hole oval (at -2.54 48.26 90) (size 1.7 1.7) (drill 1) (layers *.Cu *.Mask) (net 28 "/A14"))
  (pad "41" thru_hole oval (at 0 50.8 90) (size 1.7 1.7) (drill 1) (layers *.Cu *.Mask) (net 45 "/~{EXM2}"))
  (pad "42" thru_hole oval (at -2.54 50.8 90) (size 1.7 1.7) (drill 1) (layers *.Cu *.Mask) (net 44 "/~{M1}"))
  (pad "43" thru_hole oval (at 0 53.34 90) (size 1.7 1.7) (drill 1) (layers *.Cu *.Mask) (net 3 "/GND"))
  (pad "44" thru_hole oval (at -2.54 53.34 90) (size 1.7 1.7) (drill 1) (layers *.Cu *.Mask) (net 3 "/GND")))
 (gr_rect (start 173.99 107.188) (end 185.928 117.856) (layer "F.SilkS") (width 0.15) (fill none))
 (gr_line (start 117.238 122.686) (end 117.221 72.517) (layer "Edge.Cuts") (width 0.1))
 (gr_line (start 189.238 122.686) (end 189.23 72.517) (layer "Edge.Cuts") (width 0.1))
 (gr_line (start 117.221 72.517) (end 189.23 72.517) (layer "Edge.Cuts") (width 0.1))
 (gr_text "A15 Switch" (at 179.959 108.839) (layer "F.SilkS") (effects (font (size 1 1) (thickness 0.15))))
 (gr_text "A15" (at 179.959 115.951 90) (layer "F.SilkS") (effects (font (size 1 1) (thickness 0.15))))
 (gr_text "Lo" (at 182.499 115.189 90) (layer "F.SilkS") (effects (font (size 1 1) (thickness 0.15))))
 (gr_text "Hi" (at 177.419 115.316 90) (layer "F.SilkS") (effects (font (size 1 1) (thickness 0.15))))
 (segment (start 128.886 94.3265) (end 128.886 90.009) (width 0.25) (layer "F.Cu") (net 1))
 (segment (start 177.434 112.395) (end 177.434 101.625) (width 0.75) (layer "F.Cu") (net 1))
 (segment (start 128.886 90.009) (end 126.395 87.518) (width 0.25) (layer "F.Cu") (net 1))
 (segment (start 177.434 101.625) (end 177.459 101.6) (width 0.75) (layer "F.Cu") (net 1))
 (segment (start 161.906 109.5665) (end 174.6055 109.5665) (width 0.75) (layer "B.Cu") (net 1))
 (segment (start 174.6055 109.5665) (end 177.434 112.395) (width 0.75) (layer "B.Cu") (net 1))
 (segment (start 182.514 114.92) (end 182.514 112.395) (width 0.75) (layer "F.Cu") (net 3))
 (segment (start 183.338 115.774) (end 182.499 114.935) (width 0.75) (layer "F.Cu") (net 3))
 (segment (start 183.338 128.086) (end 183.338 115.774) (width 0.75) (layer "F.Cu") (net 3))
 (segment (start 182.514 112.395) (end 182.514 101.655) (width 0.75) (layer "F.Cu") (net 3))
 (segment (start 182.514 101.655) (end 182.459 101.6) (width 0.75) (layer "F.Cu") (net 3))
 (segment (start 182.499 114.935) (end 182.514 114.92) (width 0.75) (layer "F.Cu") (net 3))
 (segment (start 122.918 89.695) (end 122.918 128.086) (width 0.25) (layer "F.Cu") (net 29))
 (segment (start 125.095 87.518) (end 122.918 89.695) (width 0.25) (layer "F.Cu") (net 29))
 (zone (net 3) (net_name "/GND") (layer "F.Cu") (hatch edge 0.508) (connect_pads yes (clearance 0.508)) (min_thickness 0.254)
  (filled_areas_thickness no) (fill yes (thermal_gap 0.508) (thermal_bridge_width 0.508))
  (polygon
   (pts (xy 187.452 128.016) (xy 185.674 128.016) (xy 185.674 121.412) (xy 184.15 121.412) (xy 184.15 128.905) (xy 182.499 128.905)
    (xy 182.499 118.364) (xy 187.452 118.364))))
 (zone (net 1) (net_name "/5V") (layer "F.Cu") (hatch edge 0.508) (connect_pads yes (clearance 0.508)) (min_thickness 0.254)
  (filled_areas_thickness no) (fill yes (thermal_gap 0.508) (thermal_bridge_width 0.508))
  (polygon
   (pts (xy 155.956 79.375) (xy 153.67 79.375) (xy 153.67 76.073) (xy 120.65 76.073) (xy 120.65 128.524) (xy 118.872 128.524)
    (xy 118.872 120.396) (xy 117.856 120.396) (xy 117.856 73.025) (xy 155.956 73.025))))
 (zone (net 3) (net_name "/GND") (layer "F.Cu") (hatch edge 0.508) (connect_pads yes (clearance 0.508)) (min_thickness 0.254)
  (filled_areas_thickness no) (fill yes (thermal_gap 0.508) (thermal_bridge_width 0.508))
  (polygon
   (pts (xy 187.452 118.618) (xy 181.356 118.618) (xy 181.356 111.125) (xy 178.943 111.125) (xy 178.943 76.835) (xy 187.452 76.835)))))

